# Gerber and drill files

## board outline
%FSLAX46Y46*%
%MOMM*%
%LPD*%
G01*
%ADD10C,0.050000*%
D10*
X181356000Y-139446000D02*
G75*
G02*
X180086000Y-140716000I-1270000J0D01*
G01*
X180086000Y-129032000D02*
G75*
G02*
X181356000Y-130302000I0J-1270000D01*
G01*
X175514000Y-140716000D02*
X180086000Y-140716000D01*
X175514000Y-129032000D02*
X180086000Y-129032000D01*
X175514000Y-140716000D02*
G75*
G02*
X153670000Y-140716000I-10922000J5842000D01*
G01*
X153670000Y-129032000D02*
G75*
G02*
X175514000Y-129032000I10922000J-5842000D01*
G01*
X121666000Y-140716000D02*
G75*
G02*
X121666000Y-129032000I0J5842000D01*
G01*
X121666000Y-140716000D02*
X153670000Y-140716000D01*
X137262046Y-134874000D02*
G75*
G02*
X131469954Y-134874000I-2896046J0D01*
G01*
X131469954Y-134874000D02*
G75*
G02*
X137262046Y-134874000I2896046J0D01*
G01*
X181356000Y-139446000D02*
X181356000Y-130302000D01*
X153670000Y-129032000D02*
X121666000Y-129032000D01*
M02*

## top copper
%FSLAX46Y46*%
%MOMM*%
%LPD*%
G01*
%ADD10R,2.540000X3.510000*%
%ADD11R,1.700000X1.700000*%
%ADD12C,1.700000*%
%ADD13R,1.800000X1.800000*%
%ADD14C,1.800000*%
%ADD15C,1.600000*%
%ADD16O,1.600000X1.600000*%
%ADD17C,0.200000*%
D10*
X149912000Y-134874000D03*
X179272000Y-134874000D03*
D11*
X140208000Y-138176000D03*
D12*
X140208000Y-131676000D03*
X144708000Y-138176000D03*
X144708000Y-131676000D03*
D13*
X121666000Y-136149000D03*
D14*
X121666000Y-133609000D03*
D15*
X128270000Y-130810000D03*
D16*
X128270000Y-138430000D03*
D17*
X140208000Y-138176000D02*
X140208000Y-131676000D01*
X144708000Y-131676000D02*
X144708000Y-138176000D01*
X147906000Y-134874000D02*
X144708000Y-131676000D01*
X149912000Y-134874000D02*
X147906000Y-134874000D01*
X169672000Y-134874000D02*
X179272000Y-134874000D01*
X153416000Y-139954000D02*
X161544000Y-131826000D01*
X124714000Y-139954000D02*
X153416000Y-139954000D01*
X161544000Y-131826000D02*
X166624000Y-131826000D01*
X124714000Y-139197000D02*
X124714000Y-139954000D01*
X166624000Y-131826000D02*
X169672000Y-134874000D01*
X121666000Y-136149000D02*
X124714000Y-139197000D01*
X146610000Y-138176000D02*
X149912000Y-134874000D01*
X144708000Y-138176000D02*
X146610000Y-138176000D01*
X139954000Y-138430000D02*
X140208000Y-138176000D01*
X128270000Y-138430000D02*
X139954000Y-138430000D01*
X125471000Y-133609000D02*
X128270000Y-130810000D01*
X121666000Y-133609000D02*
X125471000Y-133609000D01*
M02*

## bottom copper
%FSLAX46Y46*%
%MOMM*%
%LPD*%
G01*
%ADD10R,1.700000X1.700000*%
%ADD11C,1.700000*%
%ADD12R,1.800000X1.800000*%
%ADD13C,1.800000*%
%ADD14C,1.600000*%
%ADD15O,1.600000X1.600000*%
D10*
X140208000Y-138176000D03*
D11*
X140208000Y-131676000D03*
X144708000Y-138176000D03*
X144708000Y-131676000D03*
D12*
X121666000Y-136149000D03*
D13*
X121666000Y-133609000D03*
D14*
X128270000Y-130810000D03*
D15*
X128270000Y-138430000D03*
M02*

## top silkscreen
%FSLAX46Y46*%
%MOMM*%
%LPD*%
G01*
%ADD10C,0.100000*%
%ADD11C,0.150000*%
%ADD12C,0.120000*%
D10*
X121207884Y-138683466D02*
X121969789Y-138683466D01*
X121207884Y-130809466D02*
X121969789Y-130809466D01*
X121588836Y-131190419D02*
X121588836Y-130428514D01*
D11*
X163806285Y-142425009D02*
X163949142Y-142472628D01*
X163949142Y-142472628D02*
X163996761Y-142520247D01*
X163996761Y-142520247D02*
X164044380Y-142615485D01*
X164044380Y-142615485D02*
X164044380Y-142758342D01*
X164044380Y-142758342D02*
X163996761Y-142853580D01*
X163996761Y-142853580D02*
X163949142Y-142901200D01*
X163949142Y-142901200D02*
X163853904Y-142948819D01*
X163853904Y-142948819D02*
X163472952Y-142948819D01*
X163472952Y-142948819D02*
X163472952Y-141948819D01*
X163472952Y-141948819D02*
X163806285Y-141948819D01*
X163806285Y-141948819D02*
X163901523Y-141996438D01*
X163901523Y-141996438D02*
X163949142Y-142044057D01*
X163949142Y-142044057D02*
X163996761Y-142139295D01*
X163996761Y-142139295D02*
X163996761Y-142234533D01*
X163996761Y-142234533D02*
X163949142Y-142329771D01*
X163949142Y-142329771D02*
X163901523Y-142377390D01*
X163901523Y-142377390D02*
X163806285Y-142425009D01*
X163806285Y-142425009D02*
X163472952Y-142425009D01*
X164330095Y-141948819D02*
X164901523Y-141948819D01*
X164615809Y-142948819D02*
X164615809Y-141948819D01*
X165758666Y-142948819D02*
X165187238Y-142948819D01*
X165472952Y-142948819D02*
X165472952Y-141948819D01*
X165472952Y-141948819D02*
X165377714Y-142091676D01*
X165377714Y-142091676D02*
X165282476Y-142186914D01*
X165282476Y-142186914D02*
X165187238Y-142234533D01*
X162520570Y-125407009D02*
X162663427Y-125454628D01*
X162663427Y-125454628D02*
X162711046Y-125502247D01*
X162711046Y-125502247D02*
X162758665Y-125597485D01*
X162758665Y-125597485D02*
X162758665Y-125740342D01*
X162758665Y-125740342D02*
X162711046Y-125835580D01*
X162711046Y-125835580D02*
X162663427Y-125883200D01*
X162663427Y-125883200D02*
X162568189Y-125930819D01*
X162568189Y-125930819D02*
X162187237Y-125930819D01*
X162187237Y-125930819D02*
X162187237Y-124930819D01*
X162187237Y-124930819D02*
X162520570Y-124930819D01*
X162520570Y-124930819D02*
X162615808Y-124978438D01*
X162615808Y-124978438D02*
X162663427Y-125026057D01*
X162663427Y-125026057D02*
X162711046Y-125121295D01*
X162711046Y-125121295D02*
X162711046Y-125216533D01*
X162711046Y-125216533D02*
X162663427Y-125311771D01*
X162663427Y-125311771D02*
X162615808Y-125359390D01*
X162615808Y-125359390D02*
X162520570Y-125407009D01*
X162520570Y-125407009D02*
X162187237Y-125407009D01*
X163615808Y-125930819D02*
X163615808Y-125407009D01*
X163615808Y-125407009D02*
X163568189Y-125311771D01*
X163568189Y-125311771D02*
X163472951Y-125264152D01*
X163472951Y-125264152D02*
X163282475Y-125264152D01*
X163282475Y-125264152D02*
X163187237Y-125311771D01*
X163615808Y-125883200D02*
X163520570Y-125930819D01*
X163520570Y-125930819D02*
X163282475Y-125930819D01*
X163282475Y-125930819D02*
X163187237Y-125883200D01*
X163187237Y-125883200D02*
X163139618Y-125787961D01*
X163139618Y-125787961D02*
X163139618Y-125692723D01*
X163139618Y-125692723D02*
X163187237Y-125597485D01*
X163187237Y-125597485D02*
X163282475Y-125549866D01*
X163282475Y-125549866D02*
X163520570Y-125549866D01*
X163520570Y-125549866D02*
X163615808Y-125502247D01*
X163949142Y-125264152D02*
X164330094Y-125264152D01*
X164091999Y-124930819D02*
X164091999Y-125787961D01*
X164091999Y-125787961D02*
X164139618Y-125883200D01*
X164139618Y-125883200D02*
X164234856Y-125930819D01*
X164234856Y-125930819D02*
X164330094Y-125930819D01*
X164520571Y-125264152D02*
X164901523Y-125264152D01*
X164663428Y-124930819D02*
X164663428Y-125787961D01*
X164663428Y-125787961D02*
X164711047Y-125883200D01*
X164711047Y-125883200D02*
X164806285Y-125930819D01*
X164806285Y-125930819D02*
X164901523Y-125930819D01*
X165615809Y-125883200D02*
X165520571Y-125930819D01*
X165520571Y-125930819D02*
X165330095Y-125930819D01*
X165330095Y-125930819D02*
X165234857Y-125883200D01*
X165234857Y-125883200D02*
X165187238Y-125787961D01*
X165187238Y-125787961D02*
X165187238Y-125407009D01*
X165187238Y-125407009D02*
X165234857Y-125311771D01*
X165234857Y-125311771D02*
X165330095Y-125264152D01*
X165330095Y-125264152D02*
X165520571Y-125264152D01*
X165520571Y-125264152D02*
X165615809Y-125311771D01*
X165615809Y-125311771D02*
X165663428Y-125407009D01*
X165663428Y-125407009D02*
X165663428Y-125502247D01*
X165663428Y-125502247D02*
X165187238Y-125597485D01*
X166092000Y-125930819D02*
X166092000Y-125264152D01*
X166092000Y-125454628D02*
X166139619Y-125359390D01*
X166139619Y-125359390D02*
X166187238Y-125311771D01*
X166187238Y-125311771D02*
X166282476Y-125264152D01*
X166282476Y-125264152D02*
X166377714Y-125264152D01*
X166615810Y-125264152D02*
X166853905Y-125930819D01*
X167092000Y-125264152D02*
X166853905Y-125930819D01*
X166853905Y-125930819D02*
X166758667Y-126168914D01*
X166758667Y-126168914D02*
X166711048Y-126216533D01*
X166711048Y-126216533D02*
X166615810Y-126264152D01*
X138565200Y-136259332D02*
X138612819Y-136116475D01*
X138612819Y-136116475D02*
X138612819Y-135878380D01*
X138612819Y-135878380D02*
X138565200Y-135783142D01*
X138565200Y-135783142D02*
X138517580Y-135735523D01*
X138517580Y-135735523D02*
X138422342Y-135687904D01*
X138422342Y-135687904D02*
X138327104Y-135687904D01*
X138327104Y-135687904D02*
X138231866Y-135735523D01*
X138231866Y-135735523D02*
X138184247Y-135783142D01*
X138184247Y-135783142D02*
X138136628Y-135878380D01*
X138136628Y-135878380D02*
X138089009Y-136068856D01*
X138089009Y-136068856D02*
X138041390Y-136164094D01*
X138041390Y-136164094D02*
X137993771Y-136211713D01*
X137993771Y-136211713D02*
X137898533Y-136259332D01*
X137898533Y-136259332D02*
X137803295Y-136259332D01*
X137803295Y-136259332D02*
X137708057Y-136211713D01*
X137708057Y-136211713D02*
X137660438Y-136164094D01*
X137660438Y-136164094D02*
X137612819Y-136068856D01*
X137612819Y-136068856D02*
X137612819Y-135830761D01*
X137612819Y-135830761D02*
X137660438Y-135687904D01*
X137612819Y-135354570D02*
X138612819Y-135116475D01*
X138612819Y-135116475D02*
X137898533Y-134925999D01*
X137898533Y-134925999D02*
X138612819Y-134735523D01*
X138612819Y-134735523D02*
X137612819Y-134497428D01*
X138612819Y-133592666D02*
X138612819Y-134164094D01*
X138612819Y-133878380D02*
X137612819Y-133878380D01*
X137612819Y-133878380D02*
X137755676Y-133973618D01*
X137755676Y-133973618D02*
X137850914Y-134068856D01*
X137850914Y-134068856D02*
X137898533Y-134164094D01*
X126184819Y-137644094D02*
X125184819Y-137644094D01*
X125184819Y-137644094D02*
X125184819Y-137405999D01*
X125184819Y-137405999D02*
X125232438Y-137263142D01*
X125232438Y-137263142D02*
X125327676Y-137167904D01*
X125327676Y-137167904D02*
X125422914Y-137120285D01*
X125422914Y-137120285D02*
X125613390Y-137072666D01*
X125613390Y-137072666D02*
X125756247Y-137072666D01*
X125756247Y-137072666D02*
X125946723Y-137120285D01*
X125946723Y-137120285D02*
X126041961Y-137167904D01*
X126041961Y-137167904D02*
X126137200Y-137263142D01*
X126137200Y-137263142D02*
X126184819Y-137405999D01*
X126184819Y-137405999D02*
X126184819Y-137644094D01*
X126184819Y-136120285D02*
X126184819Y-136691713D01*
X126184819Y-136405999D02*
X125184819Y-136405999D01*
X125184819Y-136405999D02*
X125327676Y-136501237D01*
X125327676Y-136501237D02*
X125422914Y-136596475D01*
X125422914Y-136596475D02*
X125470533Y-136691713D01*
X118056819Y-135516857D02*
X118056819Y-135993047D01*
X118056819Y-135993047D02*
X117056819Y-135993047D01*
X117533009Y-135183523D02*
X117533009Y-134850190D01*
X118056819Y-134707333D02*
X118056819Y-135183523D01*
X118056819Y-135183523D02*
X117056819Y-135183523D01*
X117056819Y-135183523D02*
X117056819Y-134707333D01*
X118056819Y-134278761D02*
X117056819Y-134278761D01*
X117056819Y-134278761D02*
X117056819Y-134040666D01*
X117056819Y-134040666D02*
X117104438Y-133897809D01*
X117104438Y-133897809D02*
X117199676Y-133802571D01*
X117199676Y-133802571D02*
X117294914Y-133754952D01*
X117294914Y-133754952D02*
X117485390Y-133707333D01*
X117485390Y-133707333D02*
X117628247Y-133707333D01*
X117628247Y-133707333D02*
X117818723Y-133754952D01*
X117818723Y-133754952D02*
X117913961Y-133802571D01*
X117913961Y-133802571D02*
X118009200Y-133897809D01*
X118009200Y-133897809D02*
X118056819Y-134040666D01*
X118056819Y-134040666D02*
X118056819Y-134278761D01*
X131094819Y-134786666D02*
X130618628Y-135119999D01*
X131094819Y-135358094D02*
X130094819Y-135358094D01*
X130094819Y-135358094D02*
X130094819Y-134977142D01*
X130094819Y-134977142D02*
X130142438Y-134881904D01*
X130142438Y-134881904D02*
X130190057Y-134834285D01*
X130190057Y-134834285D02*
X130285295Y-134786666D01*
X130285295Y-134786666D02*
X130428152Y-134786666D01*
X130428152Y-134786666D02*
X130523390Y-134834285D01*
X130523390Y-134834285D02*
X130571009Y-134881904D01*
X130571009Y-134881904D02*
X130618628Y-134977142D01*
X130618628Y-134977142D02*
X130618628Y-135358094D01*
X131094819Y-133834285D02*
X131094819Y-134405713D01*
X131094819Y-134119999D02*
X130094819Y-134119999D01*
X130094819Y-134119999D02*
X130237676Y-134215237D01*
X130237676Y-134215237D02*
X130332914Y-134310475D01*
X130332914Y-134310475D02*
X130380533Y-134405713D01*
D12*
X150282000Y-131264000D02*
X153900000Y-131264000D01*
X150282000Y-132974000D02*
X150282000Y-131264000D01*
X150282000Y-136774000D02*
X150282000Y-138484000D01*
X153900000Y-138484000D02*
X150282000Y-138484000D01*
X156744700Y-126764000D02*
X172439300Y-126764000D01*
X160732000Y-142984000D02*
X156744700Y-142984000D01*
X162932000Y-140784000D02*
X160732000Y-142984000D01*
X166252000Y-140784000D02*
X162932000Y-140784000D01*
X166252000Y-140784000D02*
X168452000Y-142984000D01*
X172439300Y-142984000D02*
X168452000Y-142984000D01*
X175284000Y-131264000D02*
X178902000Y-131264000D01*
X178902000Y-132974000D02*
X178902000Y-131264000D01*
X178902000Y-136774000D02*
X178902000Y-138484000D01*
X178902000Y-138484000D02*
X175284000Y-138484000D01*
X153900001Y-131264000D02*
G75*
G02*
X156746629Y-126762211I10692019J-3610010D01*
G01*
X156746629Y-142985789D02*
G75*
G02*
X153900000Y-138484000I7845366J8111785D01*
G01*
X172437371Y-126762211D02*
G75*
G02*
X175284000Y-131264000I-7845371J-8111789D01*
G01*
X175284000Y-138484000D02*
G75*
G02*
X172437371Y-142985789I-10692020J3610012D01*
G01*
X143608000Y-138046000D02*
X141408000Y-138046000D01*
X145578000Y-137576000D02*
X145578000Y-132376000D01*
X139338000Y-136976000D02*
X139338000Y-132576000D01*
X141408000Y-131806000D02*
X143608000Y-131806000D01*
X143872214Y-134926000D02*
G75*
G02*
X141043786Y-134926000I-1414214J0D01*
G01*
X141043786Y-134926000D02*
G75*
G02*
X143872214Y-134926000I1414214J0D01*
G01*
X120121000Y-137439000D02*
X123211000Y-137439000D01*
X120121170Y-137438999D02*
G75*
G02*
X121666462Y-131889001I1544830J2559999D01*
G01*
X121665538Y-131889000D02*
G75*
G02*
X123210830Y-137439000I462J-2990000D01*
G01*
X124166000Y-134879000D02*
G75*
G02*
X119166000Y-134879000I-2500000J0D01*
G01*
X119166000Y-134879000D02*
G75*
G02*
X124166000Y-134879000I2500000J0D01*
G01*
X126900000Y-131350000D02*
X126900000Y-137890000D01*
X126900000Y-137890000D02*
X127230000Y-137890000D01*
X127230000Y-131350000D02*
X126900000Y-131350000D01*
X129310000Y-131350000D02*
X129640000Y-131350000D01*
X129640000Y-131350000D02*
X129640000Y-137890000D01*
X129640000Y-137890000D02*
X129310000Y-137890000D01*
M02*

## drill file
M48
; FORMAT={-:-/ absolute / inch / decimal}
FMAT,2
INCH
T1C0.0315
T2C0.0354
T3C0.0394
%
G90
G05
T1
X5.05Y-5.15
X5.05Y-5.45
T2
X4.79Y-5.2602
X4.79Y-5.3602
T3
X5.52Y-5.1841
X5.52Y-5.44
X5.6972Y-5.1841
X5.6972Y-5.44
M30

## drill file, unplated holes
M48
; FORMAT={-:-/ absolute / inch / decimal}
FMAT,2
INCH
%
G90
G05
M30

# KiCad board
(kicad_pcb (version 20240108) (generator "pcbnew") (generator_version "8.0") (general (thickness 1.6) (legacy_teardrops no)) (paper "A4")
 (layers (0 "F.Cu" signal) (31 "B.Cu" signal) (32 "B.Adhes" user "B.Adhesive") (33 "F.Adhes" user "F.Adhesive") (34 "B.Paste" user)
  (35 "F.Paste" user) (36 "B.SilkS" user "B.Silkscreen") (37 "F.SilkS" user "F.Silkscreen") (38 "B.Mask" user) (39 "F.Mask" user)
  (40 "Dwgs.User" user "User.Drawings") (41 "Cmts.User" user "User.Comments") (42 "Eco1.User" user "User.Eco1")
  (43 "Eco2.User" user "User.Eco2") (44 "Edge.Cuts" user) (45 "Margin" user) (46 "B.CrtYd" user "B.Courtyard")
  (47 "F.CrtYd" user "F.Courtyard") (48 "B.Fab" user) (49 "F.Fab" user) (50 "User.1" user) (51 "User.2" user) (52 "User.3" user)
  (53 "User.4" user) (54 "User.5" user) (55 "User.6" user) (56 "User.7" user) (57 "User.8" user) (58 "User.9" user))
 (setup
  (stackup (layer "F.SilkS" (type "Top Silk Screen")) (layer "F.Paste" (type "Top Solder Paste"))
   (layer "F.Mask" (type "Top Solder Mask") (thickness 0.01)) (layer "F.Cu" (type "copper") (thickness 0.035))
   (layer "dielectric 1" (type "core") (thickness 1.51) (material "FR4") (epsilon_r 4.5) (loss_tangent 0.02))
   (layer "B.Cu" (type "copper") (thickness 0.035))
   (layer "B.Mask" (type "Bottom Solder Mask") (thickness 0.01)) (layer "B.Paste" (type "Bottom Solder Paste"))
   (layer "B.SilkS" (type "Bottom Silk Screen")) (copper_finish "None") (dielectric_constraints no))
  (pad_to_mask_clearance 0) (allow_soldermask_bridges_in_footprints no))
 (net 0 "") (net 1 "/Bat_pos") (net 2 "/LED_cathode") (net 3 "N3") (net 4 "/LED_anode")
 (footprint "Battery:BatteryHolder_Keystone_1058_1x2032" (layer "F.Cu") (at 164.592 134.874)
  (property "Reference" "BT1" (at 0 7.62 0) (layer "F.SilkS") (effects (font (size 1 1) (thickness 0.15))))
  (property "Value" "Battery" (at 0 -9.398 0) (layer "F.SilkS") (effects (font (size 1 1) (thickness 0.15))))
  (fp_line (start -14.31 -3.61) (end -10.692 -3.61) (stroke (width 0.12) (type solid)) (layer "F.SilkS"))
  (fp_line (start -14.31 -1.9) (end -14.31 -3.61) (stroke (width 0.12) (type solid)) (layer "F.SilkS"))
  (fp_line (start -14.31 1.9) (end -14.31 3.61) (stroke (width 0.12) (type solid)) (layer "F.SilkS"))
  (fp_line (start -10.692 3.61) (end -14.31 3.61) (stroke (width 0.12) (type solid)) (layer "F.SilkS"))
  (fp_line (start -7.8473 -8.11) (end 7.8473 -8.11) (stroke (width 0.12) (type solid)) (layer "F.SilkS"))
  (fp_line (start -3.86 8.11) (end -7.8473 8.11) (stroke (width 0.12) (type solid)) (layer "F.SilkS"))
  (fp_line (start -1.66 5.91) (end -3.86 8.11) (stroke (width 0.12) (type solid)) (layer "F.SilkS"))
  (fp_line (start 1.66 5.91) (end -1.66 5.91) (stroke (width 0.12) (type solid)) (layer "F.SilkS"))
  (fp_line (start 1.66 5.91) (end 3.86 8.11) (stroke (width 0.12) (type solid)) (layer "F.SilkS"))
  (fp_line (start 7.8473 8.11) (end 3.86 8.11) (stroke (width 0.12) (type solid)) (layer "F.SilkS"))
  (fp_line (start 10.692 -3.61) (end 14.31 -3.61) (stroke (width 0.12) (type solid)) (layer "F.SilkS"))
  (fp_line (start 14.31 -1.9) (end 14.31 -3.61) (stroke (width 0.12) (type solid)) (layer "F.SilkS"))
  (fp_line (start 14.31 1.9) (end 14.31 3.61) (stroke (width 0.12) (type solid)) (layer "F.SilkS"))
  (fp_line (start 14.31 3.61) (end 10.692 3.61) (stroke (width 0.12) (type solid)) (layer "F.SilkS"))
  (fp_arc (start -10.692 -3.61) (mid -9.538084 -6.031244) (end -7.845371 -8.111789) (stroke (width 0.12) (type solid)) (layer "F.SilkS"))
  (fp_arc (start -7.845371 8.111789) (mid -9.538085 6.031244) (end -10.692 3.61) (stroke (width 0.12) (type solid)) (layer "F.SilkS"))
  (fp_arc (start 7.845371 -8.111789) (mid 9.538085 -6.031244) (end 10.692 -3.61) (stroke (width 0.12) (type solid)) (layer "F.SilkS"))
  (fp_arc (start 10.692 3.61) (mid 9.538084 6.031244) (end 7.845371 8.111789) (stroke (width 0.12) (type solid)) (layer "F.SilkS"))
  (pad "1" smd rect (at -14.68 0) (size 2.54 3.51) (layers "F.Cu" "F.Paste" "F.Mask") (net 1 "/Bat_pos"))
  (pad "2" smd rect (at 14.68 0) (size 2.54 3.51) (layers "F.Cu" "F.Paste" "F.Mask") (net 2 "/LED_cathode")))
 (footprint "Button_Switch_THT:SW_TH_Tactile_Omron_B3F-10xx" (layer "F.Cu") (at 140.208 138.176 90)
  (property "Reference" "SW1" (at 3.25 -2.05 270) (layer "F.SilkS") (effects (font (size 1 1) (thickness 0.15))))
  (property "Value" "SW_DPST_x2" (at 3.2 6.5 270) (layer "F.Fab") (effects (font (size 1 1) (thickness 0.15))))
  (fp_line (start 1.2 -0.87) (end 5.6 -0.87) (stroke (width 0.12) (type solid)) (layer "F.SilkS"))
  (fp_line (start 6.37 1.2) (end 6.37 3.4) (stroke (width 0.12) (type solid)) (layer "F.SilkS"))
  (fp_line (start 0.13 3.4) (end 0.13 1.2) (stroke (width 0.12) (type solid)) (layer "F.SilkS"))
  (fp_line (start 0.6 5.37) (end 5.8 5.37) (stroke (width 0.12) (type solid)) (layer "F.SilkS"))
  (fp_circle (center 3.25 2.25) (end 4.25 3.25) (stroke (width 0.12) (type solid)) (fill none) (layer "F.SilkS"))
  (pad "1" thru_hole rect (at 0 0 90) (size 1.7 1.7) (drill 1) (layers "*.Cu" "*.Mask") (remove_unused_layers no) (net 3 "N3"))
  (pad "1" thru_hole circle (at 6.5 0 90) (size 1.7 1.7) (drill 1) (layers "*.Cu" "*.Mask") (remove_unused_layers no) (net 3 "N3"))
  (pad "2" thru_hole circle (at 0 4.5 90) (size 1.7 1.7) (drill 1) (layers "*.Cu" "*.Mask") (remove_unused_layers no) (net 1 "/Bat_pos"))
  (pad "2" thru_hole circle (at 6.5 4.5 90) (size 1.7 1.7) (drill 1) (layers "*.Cu" "*.Mask") (remove_unused_layers no) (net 1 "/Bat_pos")))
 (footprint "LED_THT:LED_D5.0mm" (layer "F.Cu") (at 121.666 136.149 90)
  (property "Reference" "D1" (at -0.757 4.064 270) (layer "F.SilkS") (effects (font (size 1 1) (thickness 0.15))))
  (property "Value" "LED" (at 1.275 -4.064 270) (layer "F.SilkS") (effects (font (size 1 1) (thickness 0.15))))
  (fp_line (start -1.29 -1.545) (end -1.29 1.545) (stroke (width 0.12) (type solid)) (layer "F.SilkS"))
  (fp_arc (start -1.29 -1.54483) (mid 2.072002 -2.880433) (end 4.26 0.000462) (stroke (width 0.12) (type solid)) (layer "F.SilkS"))
  (fp_arc (start 4.26 -0.000462) (mid 2.072002 2.880433) (end -1.29 1.54483) (stroke (width 0.12) (type solid)) (layer "F.SilkS"))
  (fp_circle (center 1.27 0) (end 3.77 0) (stroke (width 0.12) (type solid)) (fill none) (layer "F.SilkS"))
  (pad "1" thru_hole rect (at 0 0 90) (size 1.8 1.8) (drill 0.9) (layers "*.Cu" "*.Mask") (remove_unused_layers no) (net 2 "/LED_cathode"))
  (pad "2" thru_hole circle (at 2.54 0 90) (size 1.8 1.8) (drill 0.9) (layers "*.Cu" "*.Mask") (remove_unused_layers no)
   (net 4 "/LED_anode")))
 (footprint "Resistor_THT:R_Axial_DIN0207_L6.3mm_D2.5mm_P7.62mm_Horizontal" (layer "F.Cu") (at 128.27 130.81 -90)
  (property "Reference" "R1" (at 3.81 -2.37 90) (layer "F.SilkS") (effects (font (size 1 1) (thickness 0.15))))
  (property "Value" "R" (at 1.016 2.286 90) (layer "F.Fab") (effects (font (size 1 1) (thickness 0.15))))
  (fp_line (start 0.54 1.37) (end 7.08 1.37) (stroke (width 0.12) (type solid)) (layer "F.SilkS"))
  (fp_line (start 7.08 1.37) (end 7.08 1.04) (stroke (width 0.12) (type solid)) (layer "F.SilkS"))
  (fp_line (start 0.54 1.04) (end 0.54 1.37) (stroke (width 0.12) (type solid)) (layer "F.SilkS"))
  (fp_line (start 0.54 -1.04) (end 0.54 -1.37) (stroke (width 0.12) (type solid)) (layer "F.SilkS"))
  (fp_line (start 0.54 -1.37) (end 7.08 -1.37) (stroke (width 0.12) (type solid)) (layer "F.SilkS"))
  (fp_line (start 7.08 -1.37) (end 7.08 -1.04) (stroke (width 0.12) (type solid)) (layer "F.SilkS"))
  (pad "1" thru_hole circle (at 0 0 270) (size 1.6 1.6) (drill 0.8) (layers "*.Cu" "*.Mask") (remove_unused_layers no) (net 4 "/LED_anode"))
  (pad "2" thru_hole oval (at 7.62 0 270) (size 1.6 1.6) (drill 0.8) (layers "*.Cu" "*.Mask") (remove_unused_layers no) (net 3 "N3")))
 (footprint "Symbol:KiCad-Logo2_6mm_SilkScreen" (layer "B.Cu") (at 164.846 133.858 180)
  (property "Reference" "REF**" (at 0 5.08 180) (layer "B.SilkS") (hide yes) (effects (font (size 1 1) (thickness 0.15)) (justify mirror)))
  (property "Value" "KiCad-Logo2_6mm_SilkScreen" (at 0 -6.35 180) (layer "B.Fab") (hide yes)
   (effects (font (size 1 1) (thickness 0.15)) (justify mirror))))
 (gr_line (start 121.666 140.716) (end 153.67 140.716) (stroke (width 0.05) (type default)) (layer "Edge.Cuts"))
 (gr_line (start 175.514 129.032) (end 180.086 129.032) (stroke (width 0.05) (type default)) (layer "Edge.Cuts"))
 (gr_arc (start 181.356 139.446) (mid 180.984026 140.344026) (end 180.086 140.716) (stroke (width 0.05) (type default)) (layer "Edge.Cuts"))
 (gr_circle (center 134.366 134.874) (end 136.652 136.652) (stroke (width 0.05) (type default)) (fill none) (layer "Edge.Cuts"))
 (gr_arc (start 180.086 129.032) (mid 180.984026 129.403974) (end 181.356 130.302) (stroke (width 0.05) (type default)) (layer "Edge.Cuts"))
 (gr_arc (start 175.514 140.716) (mid 164.592 147.260244) (end 153.67 140.716) (stroke (width 0.05) (type default)) (layer "Edge.Cuts"))
 (gr_arc (start 121.666 140.716) (mid 115.824 134.874) (end 121.666 129.032) (stroke (width 0.05) (type default)) (layer "Edge.Cuts"))
 (gr_arc (start 153.67 129.032) (mid 164.592 122.487756) (end 175.514 129.032) (stroke (width 0.05) (type default)) (layer "Edge.Cuts"))
 (gr_line (start 181.356 139.446) (end 181.356 130.302) (stroke (width 0.05) (type default)) (layer "Edge.Cuts"))
 (gr_line (start 153.67 129.032) (end 121.666 129.032) (stroke (width 0.05) (type default)) (layer "Edge.Cuts"))
 (gr_line (start 175.514 140.716) (end 180.086 140.716) (stroke (width 0.05) (type default)) (layer "Edge.Cuts"))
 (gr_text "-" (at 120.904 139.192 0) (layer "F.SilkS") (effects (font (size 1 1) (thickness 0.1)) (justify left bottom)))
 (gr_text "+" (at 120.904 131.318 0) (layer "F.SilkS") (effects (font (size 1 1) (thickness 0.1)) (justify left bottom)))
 (segment (start 121.666 136.149) (end 124.714 139.197) (width 0.2) (layer "F.Cu") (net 2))
 (segment (start 124.714 139.954) (end 153.416 139.954) (width 0.2) (layer "F.Cu") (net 2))
 (segment (start 124.714 139.197) (end 124.714 139.954) (width 0.2) (layer "F.Cu") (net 2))
 (segment (start 161.544 131.826) (end 166.624 131.826) (width 0.2) (layer "F.Cu") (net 2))
 (segment (start 153.416 139.954) (end 161.544 131.826) (width 0.2) (layer "F.Cu") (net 2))
 (segment (start 169.672 134.874) (end 179.272 134.874) (width 0.2) (layer "F.Cu") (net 2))
 (segment (start 166.624 131.826) (end 169.672 134.874) (width 0.2) (layer "F.Cu") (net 2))
 (segment (start 149.912 134.874) (end 147.906 134.874) (width 0.2) (layer "F.Cu") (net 1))
 (segment (start 144.708 138.176) (end 146.61 138.176) (width 0.2) (layer "F.Cu") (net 1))
 (segment (start 144.708 131.676) (end 144.708 138.176) (width 0.2) (layer "F.Cu") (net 1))
 (segment (start 146.61 138.176) (end 149.912 134.874) (width 0.2) (layer "F.Cu") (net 1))
 (segment (start 147.906 134.874) (end 144.708 131.676) (width 0.2) (layer "F.Cu") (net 1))
 (segment (start 125.471 133.609) (end 128.27 130.81) (width 0.2) (layer "F.Cu") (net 4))
 (segment (start 121.666 133.609) (end 125.471 133.609) (width 0.2) (layer "F.Cu") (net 4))
 (segment (start 139.954 138.43) (end 140.208 138.176) (width 0.2) (layer "F.Cu") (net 3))
 (segment (start 140.208 138.176) (end 140.208 131.676) (width 0.2) (layer "F.Cu") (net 3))
 (segment (start 128.27 138.43) (end 139.954 138.43) (width 0.2) (layer "F.Cu") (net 3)))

